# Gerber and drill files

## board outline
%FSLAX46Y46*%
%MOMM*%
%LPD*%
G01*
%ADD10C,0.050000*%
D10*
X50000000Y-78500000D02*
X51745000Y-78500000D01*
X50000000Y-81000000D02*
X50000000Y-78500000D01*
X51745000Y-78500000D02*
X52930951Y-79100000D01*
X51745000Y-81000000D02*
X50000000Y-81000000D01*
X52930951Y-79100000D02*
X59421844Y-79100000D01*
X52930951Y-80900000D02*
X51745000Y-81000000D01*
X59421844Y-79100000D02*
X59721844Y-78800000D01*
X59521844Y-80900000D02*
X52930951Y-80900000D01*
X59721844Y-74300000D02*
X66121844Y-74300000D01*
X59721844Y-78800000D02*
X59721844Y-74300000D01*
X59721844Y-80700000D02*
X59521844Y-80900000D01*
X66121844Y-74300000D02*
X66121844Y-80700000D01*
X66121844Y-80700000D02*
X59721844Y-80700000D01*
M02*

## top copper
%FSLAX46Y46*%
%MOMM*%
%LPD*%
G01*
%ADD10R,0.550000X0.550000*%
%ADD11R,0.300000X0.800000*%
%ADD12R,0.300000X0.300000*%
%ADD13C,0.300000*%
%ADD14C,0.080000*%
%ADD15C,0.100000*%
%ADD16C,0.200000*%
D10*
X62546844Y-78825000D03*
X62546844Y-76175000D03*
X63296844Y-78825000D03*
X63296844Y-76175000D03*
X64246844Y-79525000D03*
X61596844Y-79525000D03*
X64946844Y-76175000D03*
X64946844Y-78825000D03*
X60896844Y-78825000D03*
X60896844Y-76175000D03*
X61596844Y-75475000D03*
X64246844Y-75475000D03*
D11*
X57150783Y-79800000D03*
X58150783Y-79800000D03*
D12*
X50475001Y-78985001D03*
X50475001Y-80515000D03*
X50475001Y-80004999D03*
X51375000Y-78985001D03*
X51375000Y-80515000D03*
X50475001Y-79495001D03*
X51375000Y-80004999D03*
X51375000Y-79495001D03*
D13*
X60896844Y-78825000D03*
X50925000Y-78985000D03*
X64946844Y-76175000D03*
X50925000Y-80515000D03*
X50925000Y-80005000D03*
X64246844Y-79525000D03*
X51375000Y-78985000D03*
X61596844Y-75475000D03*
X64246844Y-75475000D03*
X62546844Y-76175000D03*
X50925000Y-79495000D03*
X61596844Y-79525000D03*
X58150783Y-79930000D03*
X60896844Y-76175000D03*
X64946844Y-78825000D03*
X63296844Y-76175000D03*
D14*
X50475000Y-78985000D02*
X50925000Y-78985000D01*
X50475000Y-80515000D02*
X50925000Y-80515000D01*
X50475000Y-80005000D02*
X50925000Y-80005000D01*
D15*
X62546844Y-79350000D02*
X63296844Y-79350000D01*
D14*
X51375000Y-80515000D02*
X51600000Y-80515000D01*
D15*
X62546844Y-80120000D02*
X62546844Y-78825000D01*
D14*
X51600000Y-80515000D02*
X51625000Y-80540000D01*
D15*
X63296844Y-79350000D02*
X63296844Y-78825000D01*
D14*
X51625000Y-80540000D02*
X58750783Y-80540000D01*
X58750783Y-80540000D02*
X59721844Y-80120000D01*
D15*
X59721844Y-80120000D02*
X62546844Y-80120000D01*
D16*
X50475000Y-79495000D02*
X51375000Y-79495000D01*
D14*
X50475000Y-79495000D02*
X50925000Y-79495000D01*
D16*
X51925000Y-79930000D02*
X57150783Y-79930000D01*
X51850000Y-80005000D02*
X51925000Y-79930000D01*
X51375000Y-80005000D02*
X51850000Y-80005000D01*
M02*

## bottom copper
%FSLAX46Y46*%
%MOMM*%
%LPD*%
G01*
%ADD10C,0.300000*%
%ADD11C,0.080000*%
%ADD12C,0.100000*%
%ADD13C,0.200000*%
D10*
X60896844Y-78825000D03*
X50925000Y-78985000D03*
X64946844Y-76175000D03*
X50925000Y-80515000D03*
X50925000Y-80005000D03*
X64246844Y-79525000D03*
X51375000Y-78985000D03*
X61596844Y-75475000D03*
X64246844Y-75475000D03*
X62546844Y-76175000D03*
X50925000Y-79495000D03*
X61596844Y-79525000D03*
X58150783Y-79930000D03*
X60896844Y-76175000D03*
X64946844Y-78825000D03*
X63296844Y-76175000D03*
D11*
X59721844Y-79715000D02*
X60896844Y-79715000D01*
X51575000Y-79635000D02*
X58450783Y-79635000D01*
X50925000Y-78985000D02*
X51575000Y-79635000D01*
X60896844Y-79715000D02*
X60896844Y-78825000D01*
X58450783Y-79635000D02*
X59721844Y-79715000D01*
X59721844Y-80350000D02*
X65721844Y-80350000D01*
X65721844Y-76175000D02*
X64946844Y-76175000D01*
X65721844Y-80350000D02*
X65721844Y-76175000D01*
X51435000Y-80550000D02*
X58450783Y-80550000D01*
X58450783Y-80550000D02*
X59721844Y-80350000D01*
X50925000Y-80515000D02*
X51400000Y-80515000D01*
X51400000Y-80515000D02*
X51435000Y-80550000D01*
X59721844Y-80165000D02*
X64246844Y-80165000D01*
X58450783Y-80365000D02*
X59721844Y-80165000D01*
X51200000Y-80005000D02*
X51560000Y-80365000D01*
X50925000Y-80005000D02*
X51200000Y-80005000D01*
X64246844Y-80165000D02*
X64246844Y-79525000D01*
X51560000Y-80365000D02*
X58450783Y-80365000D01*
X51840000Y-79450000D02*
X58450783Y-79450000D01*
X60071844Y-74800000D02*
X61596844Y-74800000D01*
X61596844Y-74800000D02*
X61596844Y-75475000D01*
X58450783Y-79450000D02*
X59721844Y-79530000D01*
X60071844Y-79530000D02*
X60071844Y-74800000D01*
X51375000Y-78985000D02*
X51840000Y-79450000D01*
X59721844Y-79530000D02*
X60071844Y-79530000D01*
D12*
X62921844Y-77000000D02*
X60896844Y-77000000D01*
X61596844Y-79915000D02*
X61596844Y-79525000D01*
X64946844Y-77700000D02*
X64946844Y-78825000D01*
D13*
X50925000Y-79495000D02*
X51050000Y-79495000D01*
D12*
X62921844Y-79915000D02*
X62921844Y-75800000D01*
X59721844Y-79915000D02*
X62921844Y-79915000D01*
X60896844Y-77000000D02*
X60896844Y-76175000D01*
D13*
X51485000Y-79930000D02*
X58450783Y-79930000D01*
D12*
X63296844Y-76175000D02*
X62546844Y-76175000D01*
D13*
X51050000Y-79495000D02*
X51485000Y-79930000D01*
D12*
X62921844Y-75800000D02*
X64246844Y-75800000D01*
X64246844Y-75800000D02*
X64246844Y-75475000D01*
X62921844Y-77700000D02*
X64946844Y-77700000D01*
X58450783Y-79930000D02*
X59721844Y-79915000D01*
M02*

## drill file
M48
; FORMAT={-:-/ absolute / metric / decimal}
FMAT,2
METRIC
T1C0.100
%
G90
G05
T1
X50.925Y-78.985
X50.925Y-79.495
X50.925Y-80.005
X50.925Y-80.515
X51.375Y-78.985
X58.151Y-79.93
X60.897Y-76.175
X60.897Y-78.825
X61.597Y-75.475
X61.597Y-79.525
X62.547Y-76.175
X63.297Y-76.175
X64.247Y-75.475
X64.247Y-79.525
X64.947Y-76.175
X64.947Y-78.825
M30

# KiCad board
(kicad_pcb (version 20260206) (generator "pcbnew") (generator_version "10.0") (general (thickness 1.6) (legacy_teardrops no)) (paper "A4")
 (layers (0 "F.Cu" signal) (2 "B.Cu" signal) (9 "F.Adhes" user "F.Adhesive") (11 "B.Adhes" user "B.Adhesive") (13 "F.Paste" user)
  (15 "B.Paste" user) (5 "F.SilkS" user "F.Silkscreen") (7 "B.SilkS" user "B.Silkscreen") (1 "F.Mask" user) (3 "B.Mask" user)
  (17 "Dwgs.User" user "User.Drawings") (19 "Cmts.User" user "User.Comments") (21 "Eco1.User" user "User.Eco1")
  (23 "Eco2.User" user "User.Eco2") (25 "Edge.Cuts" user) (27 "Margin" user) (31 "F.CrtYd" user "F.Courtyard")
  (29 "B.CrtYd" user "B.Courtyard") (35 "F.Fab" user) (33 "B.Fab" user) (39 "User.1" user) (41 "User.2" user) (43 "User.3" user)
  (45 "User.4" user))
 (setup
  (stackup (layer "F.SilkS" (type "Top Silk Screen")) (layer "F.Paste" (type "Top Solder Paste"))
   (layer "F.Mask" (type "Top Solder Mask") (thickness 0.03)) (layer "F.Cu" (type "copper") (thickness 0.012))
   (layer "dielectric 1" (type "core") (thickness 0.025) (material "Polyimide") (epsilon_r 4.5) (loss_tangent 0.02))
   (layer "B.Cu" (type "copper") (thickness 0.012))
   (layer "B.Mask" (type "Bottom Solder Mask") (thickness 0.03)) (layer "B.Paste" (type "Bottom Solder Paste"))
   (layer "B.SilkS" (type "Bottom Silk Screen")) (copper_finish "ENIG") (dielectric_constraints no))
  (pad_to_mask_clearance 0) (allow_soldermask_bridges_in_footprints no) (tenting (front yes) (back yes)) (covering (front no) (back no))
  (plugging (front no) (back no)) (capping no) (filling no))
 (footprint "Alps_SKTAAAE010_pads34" (layer "F.Cu") (at 62.921844 75.1)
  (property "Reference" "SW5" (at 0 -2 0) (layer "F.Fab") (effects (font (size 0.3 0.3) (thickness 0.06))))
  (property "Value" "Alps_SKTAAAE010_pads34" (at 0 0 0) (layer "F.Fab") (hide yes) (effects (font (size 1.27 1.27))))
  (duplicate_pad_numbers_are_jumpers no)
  (pad "3" smd rect (at -1.325 0.375) (size 0.55 0.55) (layers "F.Cu" "F.Mask" "F.Paste") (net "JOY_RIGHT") (solder_mask_margin 0.05)
   (thermal_bridge_angle 45))
  (pad "4" smd rect (at 1.325 0.375) (size 0.55 0.55) (layers "F.Cu" "F.Mask" "F.Paste") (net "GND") (solder_mask_margin 0.05)
   (thermal_bridge_angle 45)))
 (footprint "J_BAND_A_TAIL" (layer "F.Cu") (at 50.9 79.75)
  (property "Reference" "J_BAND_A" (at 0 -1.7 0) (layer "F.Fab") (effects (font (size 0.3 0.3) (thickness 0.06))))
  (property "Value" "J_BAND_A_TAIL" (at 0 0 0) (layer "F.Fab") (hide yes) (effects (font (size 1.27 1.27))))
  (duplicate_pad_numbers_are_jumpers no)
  (pad "1" smd rect (at -0.424999 -0.764999) (size 0.3 0.3) (layers "F.Cu" "F.Mask") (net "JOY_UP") (solder_mask_margin 0.05)
   (thermal_bridge_angle 45))
  (pad "2" smd rect (at -0.424999 0.765) (size 0.3 0.3) (layers "F.Cu" "F.Mask") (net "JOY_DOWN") (solder_mask_margin 0.05)
   (thermal_bridge_angle 45))
  (pad "3" smd rect (at -0.424999 0.254999) (size 0.3 0.3) (layers "F.Cu" "F.Mask") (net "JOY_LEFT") (solder_mask_margin 0.05)
   (thermal_bridge_angle 45))
  (pad "4" smd rect (at 0.475 -0.764999) (size 0.3 0.3) (layers "F.Cu" "F.Mask") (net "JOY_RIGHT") (solder_mask_margin 0.05)
   (thermal_bridge_angle 45))
  (pad "5" smd rect (at 0.475 0.765) (size 0.3 0.3) (layers "F.Cu" "F.Mask") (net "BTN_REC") (solder_mask_margin 0.05)
   (thermal_bridge_angle 45))
  (pad "6" smd rect (at -0.424999 -0.254999) (size 0.3 0.3) (layers "F.Cu" "F.Mask") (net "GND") (solder_mask_margin 0.05)
   (thermal_bridge_angle 45))
  (pad "7" smd rect (at 0.475 0.254999) (size 0.3 0.3) (layers "F.Cu" "F.Mask") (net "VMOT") (solder_mask_margin 0.05)
   (thermal_bridge_angle 45))
  (pad "8" smd rect (at 0.475 -0.254999) (size 0.3 0.3) (layers "F.Cu" "F.Mask") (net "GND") (solder_mask_margin 0.05)
   (thermal_bridge_angle 45)))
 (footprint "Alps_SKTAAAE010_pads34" (layer "F.Cu") (at 62.921844 79.9 180)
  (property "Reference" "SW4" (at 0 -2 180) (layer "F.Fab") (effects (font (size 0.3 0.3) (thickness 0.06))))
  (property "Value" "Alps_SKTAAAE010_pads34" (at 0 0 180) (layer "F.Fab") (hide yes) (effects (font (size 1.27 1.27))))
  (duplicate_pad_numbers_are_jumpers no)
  (pad "3" smd rect (at -1.325 0.375 180) (size 0.55 0.55) (layers "F.Cu" "F.Mask" "F.Paste") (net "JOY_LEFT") (solder_mask_margin 0.05)
   (thermal_bridge_angle 45))
  (pad "4" smd rect (at 1.325 0.375 180) (size 0.55 0.55) (layers "F.Cu" "F.Mask" "F.Paste") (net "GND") (solder_mask_margin 0.05)
   (thermal_bridge_angle 45)))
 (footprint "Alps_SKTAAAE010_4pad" (layer "F.Cu") (at 62.921844 77.5 90)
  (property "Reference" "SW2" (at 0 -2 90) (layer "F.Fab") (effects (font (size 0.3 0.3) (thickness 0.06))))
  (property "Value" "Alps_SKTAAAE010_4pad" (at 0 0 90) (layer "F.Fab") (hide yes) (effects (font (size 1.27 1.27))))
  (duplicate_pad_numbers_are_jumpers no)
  (pad "1" smd rect (at -1.325 -0.375 90) (size 0.55 0.55) (layers "F.Cu" "F.Mask") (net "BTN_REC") (solder_mask_margin 0.05)
   (thermal_bridge_angle 45))
  (pad "2" smd rect (at 1.325 -0.375 90) (size 0.55 0.55) (layers "F.Cu" "F.Mask" "F.Paste") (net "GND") (solder_mask_margin 0.05)
   (thermal_bridge_angle 45))
  (pad "3" smd rect (at -1.325 0.375 90) (size 0.55 0.55) (layers "F.Cu" "F.Mask" "F.Paste") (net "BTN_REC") (solder_mask_margin 0.05)
   (thermal_bridge_angle 45))
  (pad "4" smd rect (at 1.325 0.375 90) (size 0.55 0.55) (layers "F.Cu" "F.Mask" "F.Paste") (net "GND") (solder_mask_margin 0.05)
   (thermal_bridge_angle 45)))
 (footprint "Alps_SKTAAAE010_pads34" (layer "F.Cu") (at 65.321844 77.5 -90)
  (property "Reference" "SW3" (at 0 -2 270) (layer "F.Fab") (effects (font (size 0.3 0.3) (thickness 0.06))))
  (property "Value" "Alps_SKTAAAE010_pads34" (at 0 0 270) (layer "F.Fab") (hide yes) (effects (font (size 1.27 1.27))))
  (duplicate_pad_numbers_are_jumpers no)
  (pad "3" smd rect (at -1.325 0.375 270) (size 0.55 0.55) (layers "F.Cu" "F.Mask" "F.Paste") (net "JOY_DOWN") (solder_mask_margin 0.05)
   (thermal_bridge_angle 45))
  (pad "4" smd rect (at 1.325 0.375 270) (size 0.55 0.55) (layers "F.Cu" "F.Mask" "F.Paste") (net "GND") (solder_mask_margin 0.05)
   (thermal_bridge_angle 45)))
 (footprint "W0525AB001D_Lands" (layer "F.Cu") (at 57.650783 79.93)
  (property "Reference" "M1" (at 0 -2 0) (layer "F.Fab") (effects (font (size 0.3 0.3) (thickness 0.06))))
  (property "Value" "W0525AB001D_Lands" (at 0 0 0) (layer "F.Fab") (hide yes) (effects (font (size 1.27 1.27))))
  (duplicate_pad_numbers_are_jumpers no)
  (pad "1" smd rect (at -0.5 -0.13) (size 0.3 0.8) (layers "F.Cu" "F.Mask") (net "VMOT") (solder_mask_margin 0.05) (thermal_bridge_angle 45))
  (pad "2" smd rect (at 0.5 -0.13) (size 0.3 0.8) (layers "F.Cu" "F.Mask") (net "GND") (solder_mask_margin 0.05) (thermal_bridge_angle 45)))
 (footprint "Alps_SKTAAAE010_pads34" (layer "F.Cu") (at 60.521844 77.5 90)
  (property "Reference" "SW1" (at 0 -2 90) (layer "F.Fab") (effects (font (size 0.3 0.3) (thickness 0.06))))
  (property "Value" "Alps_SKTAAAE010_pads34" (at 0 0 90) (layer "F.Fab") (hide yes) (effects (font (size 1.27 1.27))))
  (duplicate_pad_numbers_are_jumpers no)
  (pad "3" smd rect (at -1.325 0.375 90) (size 0.55 0.55) (layers "F.Cu" "F.Mask" "F.Paste") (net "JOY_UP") (solder_mask_margin 0.05)
   (thermal_bridge_angle 45))
  (pad "4" smd rect (at 1.325 0.375 90) (size 0.55 0.55) (layers "F.Cu" "F.Mask" "F.Paste") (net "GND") (solder_mask_margin 0.05)
   (thermal_bridge_angle 45)))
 (gr_line (start 50 78.5) (end 51.745 78.5) (stroke (width 0.05) (type default)) (layer "Edge.Cuts"))
 (gr_line (start 50 81) (end 50 78.5) (stroke (width 0.05) (type default)) (layer "Edge.Cuts"))
 (gr_line (start 51.745 78.5) (end 52.930951 79.1) (stroke (width 0.05) (type default)) (layer "Edge.Cuts"))
 (gr_line (start 51.745 81) (end 50 81) (stroke (width 0.05) (type default)) (layer "Edge.Cuts"))
 (gr_line (start 52.930951 79.1) (end 59.421844 79.1) (stroke (width 0.05) (type default)) (layer "Edge.Cuts"))
 (gr_line (start 52.930951 80.9) (end 51.745 81) (stroke (width 0.05) (type default)) (layer "Edge.Cuts"))
 (gr_line (start 59.421844 79.1) (end 59.721844 78.8) (stroke (width 0.05) (type default)) (layer "Edge.Cuts"))
 (gr_line (start 59.521844 80.9) (end 52.930951 80.9) (stroke (width 0.05) (type default)) (layer "Edge.Cuts"))
 (gr_line (start 59.721844 74.3) (end 66.121844 74.3) (stroke (width 0.05) (type default)) (layer "Edge.Cuts"))
 (gr_line (start 59.721844 78.8) (end 59.721844 74.3) (stroke (width 0.05) (type default)) (layer "Edge.Cuts"))
 (gr_line (start 59.721844 80.7) (end 59.521844 80.9) (stroke (width 0.05) (type default)) (layer "Edge.Cuts"))
 (gr_line (start 66.121844 74.3) (end 66.121844 80.7) (stroke (width 0.05) (type default)) (layer "Edge.Cuts"))
 (gr_line (start 66.121844 80.7) (end 59.721844 80.7) (stroke (width 0.05) (type default)) (layer "Edge.Cuts"))
 (via (at 51.375 78.985) (size 0.3) (drill 0.1) (layers "F.Cu" "B.Cu") (tenting (front yes) (back yes)) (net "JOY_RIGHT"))
 (via (at 61.596844 75.475) (size 0.3) (drill 0.1) (layers "F.Cu" "B.Cu") (tenting (front yes) (back yes)) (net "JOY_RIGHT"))
 (segment (start 59.721844 79.53) (end 60.071844 79.53) (width 0.08) (layer "B.Cu") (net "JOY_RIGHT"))
 (segment (start 51.375 78.985) (end 51.84 79.45) (width 0.08) (layer "B.Cu") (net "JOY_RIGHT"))
 (segment (start 51.84 79.45) (end 58.450783 79.45) (width 0.08) (layer "B.Cu") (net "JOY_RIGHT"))
 (segment (start 58.450783 79.45) (end 59.721844 79.53) (width 0.08) (layer "B.Cu") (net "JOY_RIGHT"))
 (segment (start 61.596844 74.8) (end 61.596844 75.475) (width 0.08) (layer "B.Cu") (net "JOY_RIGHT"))
 (segment (start 60.071844 79.53) (end 60.071844 74.8) (width 0.08) (layer "B.Cu") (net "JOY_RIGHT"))
 (segment (start 60.071844 74.8) (end 61.596844 74.8) (width 0.08) (layer "B.Cu") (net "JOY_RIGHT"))
 (segment (start 50.475 79.495) (end 50.925 79.495) (width 0.08) (layer "F.Cu") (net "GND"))
 (segment (start 50.475 79.495) (end 51.375 79.495) (width 0.2) (layer "F.Cu") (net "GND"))
 (via (at 60.896844 76.175) (size 0.3) (drill 0.1) (layers "F.Cu" "B.Cu") (tenting (front yes) (back yes)) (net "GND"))
 (via (at 63.296844 76.175) (size 0.3) (drill 0.1) (layers "F.Cu" "B.Cu") (tenting (front yes) (back yes)) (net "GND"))
 (via (at 64.246844 75.475) (size 0.3) (drill 0.1) (layers "F.Cu" "B.Cu") (tenting (front yes) (back yes)) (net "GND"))
 (via (at 64.946844 78.825) (size 0.3) (drill 0.1) (layers "F.Cu" "B.Cu") (tenting (front yes) (back yes)) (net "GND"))
 (via (at 62.546844 76.175) (size 0.3) (drill 0.1) (layers "F.Cu" "B.Cu") (tenting (front yes) (back yes)) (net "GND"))
 (via (at 58.150783 79.93) (size 0.3) (drill 0.1) (layers "F.Cu" "B.Cu") (tenting (front yes) (back yes)) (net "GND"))
 (via (at 61.596844 79.525) (size 0.3) (drill 0.1) (layers "F.Cu" "B.Cu") (tenting (front yes) (back yes)) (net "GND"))
 (via (at 50.925 79.495) (size 0.3) (drill 0.1) (layers "F.Cu" "B.Cu") (tenting (front yes) (back yes)) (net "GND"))
 (segment (start 64.946844 77.7) (end 64.946844 78.825) (width 0.1) (layer "B.Cu") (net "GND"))
 (segment (start 63.296844 76.175) (end 62.546844 76.175) (width 0.1) (layer "B.Cu") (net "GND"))
 (segment (start 60.896844 77) (end 60.896844 76.175) (width 0.1) (layer "B.Cu") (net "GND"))
 (segment (start 50.925 79.495) (end 51.05 79.495) (width 0.2) (layer "B.Cu") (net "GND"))
 (segment (start 62.921844 77) (end 60.896844 77) (width 0.1) (layer "B.Cu") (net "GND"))
 (segment (start 61.596844 79.915) (end 61.596844 79.525) (width 0.1) (layer "B.Cu") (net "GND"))
 (segment (start 58.450783 79.93) (end 59.721844 79.915) (width 0.1) (layer "B.Cu") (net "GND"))
 (segment (start 51.05 79.495) (end 51.485 79.93) (width 0.2) (layer "B.Cu") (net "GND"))
 (segment (start 62.921844 75.8) (end 64.246844 75.8) (width 0.1) (layer "B.Cu") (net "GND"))
 (segment (start 64.246844 75.8) (end 64.246844 75.475) (width 0.1) (layer "B.Cu") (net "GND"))
 (segment (start 51.485 79.93) (end 58.450783 79.93) (width 0.2) (layer "B.Cu") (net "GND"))
 (segment (start 62.921844 77.7) (end 64.946844 77.7) (width 0.1) (layer "B.Cu") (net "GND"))
 (segment (start 59.721844 79.915) (end 62.921844 79.915) (width 0.1) (layer "B.Cu") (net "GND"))
 (segment (start 62.921844 79.915) (end 62.921844 75.8) (width 0.1) (layer "B.Cu") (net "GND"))
 (segment (start 50.475 78.985) (end 50.925 78.985) (width 0.08) (layer "F.Cu") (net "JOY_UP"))
 (via (at 60.896844 78.825) (size 0.3) (drill 0.1) (layers "F.Cu" "B.Cu") (tenting (front yes) (back yes)) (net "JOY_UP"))
 (via (at 50.925 78.985) (size 0.3) (drill 0.1) (layers "F.Cu" "B.Cu") (tenting (front yes) (back yes)) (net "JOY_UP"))
 (segment (start 58.450783 79.635) (end 59.721844 79.715) (width 0.08) (layer "B.Cu") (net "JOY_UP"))
 (segment (start 51.575 79.635) (end 58.450783 79.635) (width 0.08) (layer "B.Cu") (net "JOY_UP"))
 (segment (start 50.925 78.985) (end 51.575 79.635) (width 0.08) (layer "B.Cu") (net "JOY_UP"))
 (segment (start 60.896844 79.715) (end 60.896844 78.825) (width 0.08) (layer "B.Cu") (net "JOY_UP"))
 (segment (start 59.721844 79.715) (end 60.896844 79.715) (width 0.08) (layer "B.Cu") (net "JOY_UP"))
 (segment (start 50.475 80.515) (end 50.925 80.515) (width 0.08) (layer "F.Cu") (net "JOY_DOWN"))
 (via (at 50.925 80.515) (size 0.3) (drill 0.1) (layers "F.Cu" "B.Cu") (tenting (front yes) (back yes)) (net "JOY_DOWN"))
 (via (at 64.946844 76.175) (size 0.3) (drill 0.1) (layers "F.Cu" "B.Cu") (tenting (front yes) (back yes)) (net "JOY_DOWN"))
 (segment (start 59.721844 80.35) (end 65.721844 80.35) (width 0.08) (layer "B.Cu") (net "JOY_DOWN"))
 (segment (start 65.721844 76.175) (end 64.946844 76.175) (width 0.08) (layer "B.Cu") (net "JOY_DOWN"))
 (segment (start 50.925 80.515) (end 51.4 80.515) (width 0.08) (layer "B.Cu") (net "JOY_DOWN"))
 (segment (start 58.450783 80.55) (end 59.721844 80.35) (width 0.08) (layer "B.Cu") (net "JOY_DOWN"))
 (segment (start 65.721844 80.35) (end 65.721844 76.175) (width 0.08) (layer "B.Cu") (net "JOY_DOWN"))
 (segment (start 51.4 80.515) (end 51.435 80.55) (width 0.08) (layer "B.Cu") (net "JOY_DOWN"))
 (segment (start 51.435 80.55) (end 58.450783 80.55) (width 0.08) (layer "B.Cu") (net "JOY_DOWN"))
 (segment (start 50.475 80.005) (end 50.925 80.005) (width 0.08) (layer "F.Cu") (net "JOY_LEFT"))
 (via (at 64.246844 79.525) (size 0.3) (drill 0.1) (layers "F.Cu" "B.Cu") (tenting (front yes) (back yes)) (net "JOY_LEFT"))
 (via (at 50.925 80.005) (size 0.3) (drill 0.1) (layers "F.Cu" "B.Cu") (tenting (front yes) (back yes)) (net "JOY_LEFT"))
 (segment (start 51.2 80.005) (end 51.56 80.365) (width 0.08) (layer "B.Cu") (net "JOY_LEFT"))
 (segment (start 59.721844 80.165) (end 64.246844 80.165) (width 0.08) (layer "B.Cu") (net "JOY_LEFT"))
 (segment (start 64.246844 80.165) (end 64.246844 79.525) (width 0.08) (layer "B.Cu") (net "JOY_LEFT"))
 (segment (start 58.450783 80.365) (end 59.721844 80.165) (width 0.08) (layer "B.Cu") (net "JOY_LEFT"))
 (segment (start 50.925 80.005) (end 51.2 80.005) (width 0.08) (layer "B.Cu") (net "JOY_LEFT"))
 (segment (start 51.56 80.365) (end 58.450783 80.365) (width 0.08) (layer "B.Cu") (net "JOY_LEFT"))
 (segment (start 62.546844 79.35) (end 63.296844 79.35) (width 0.1) (layer "F.Cu") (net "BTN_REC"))
 (segment (start 63.296844 79.35) (end 63.296844 78.825) (width 0.1) (layer "F.Cu") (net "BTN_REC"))
 (segment (start 51.375 80.515) (end 51.6 80.515) (width 0.08) (layer "F.Cu") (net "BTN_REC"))
 (segment (start 58.750783 80.54) (end 59.721844 80.12) (width 0.08) (layer "F.Cu") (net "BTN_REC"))
 (segment (start 51.6 80.515) (end 51.625 80.54) (width 0.08) (layer "F.Cu") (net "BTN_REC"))
 (segment (start 59.721844 80.12) (end 62.546844 80.12) (width 0.1) (layer "F.Cu") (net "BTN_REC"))
 (segment (start 51.625 80.54) (end 58.750783 80.54) (width 0.08) (layer "F.Cu") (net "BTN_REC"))
 (segment (start 62.546844 80.12) (end 62.546844 78.825) (width 0.1) (layer "F.Cu") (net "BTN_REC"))
 (segment (start 51.925 79.93) (end 57.150783 79.93) (width 0.2) (layer "F.Cu") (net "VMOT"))
 (segment (start 51.375 80.005) (end 51.85 80.005) (width 0.2) (layer "F.Cu") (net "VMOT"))
 (segment (start 51.85 80.005) (end 51.925 79.93) (width 0.2) (layer "F.Cu") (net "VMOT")))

